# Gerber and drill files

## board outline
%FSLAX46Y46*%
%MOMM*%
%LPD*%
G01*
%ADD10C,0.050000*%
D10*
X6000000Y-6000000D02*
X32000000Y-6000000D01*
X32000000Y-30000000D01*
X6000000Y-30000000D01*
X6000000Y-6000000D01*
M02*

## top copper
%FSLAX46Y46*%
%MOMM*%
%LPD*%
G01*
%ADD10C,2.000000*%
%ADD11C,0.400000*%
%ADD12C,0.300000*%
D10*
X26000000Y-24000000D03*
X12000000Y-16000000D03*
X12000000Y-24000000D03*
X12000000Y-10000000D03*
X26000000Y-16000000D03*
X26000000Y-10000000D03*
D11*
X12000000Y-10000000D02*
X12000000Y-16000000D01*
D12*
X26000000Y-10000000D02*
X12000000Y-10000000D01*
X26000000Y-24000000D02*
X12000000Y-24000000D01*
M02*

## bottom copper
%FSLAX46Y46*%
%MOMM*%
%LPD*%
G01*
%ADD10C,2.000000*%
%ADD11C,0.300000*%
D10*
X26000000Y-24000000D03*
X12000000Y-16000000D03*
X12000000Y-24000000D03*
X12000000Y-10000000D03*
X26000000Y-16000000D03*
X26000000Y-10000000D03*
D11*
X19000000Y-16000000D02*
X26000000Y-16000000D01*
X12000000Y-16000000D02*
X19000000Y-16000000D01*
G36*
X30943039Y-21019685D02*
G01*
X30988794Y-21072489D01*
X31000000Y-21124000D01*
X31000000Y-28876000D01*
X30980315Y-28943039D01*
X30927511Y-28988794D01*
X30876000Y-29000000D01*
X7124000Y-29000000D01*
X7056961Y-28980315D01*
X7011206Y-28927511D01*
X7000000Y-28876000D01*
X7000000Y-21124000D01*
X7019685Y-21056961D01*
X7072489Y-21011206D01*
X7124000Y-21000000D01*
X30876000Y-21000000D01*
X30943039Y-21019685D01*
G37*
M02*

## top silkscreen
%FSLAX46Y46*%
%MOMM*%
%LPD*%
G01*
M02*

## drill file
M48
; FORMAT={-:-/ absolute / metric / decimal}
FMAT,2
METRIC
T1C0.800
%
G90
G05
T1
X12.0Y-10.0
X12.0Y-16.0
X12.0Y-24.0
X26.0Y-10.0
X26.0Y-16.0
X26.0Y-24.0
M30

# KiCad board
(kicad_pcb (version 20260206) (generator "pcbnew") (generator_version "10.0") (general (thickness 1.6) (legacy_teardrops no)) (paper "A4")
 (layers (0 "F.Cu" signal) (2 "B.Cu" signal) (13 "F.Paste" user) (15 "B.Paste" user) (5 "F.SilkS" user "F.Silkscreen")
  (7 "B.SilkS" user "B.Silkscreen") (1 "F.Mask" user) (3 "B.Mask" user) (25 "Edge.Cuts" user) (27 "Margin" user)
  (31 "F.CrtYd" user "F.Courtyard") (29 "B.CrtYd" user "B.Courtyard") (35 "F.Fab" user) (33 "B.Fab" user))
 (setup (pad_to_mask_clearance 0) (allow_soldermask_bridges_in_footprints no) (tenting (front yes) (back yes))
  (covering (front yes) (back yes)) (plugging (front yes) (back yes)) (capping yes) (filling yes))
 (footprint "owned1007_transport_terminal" (layer "F.Cu") (at 26 24)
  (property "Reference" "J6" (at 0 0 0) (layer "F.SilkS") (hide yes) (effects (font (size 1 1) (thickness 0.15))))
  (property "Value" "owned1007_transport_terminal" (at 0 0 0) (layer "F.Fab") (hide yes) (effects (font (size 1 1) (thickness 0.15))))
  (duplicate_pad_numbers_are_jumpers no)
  (pad "1" thru_hole circle (at 0 0) (size 2 2) (drill 0.8) (layers "*.Cu" "*.Mask") (remove_unused_layers no) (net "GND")))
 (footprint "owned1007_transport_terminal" (layer "F.Cu") (at 12 16)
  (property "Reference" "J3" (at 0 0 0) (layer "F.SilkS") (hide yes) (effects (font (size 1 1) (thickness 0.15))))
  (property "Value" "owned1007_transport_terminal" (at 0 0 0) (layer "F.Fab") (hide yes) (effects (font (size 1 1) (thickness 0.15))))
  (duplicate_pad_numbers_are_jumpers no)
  (pad "1" thru_hole circle (at 0 0) (size 2 2) (drill 0.8) (layers "*.Cu" "*.Mask") (remove_unused_layers no) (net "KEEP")))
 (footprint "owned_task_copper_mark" (layer "F.Cu") (at 10 28)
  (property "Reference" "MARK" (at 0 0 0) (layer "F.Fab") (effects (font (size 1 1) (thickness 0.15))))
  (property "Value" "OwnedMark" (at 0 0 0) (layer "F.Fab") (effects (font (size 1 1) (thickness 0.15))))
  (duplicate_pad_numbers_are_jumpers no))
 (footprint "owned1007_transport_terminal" (layer "F.Cu") (at 12 24)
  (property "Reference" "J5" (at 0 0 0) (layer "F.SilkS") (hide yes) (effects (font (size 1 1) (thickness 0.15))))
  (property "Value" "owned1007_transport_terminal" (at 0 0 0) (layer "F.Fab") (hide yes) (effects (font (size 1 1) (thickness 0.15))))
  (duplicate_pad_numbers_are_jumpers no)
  (pad "1" thru_hole circle (at 0 0) (size 2 2) (drill 0.8) (layers "*.Cu" "*.Mask") (remove_unused_layers no) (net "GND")))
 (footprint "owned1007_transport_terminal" (layer "F.Cu") (at 12 10)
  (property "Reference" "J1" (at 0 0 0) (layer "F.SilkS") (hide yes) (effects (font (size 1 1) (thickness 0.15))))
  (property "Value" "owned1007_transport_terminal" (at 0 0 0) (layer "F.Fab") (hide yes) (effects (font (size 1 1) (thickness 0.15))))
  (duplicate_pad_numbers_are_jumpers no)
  (pad "1" thru_hole circle (at 0 0) (size 2 2) (drill 0.8) (layers "*.Cu" "*.Mask") (remove_unused_layers no) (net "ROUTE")))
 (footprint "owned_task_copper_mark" (layer "F.Cu") (at 13 28)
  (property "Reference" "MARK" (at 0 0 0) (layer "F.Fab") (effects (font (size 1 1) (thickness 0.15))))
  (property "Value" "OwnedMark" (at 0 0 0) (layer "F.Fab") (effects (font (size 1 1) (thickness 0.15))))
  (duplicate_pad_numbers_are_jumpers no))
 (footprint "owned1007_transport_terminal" (layer "F.Cu") (at 26 16)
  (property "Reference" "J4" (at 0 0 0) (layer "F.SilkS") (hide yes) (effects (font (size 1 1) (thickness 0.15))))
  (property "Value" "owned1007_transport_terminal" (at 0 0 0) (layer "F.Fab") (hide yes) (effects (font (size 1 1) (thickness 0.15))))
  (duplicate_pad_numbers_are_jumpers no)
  (pad "1" thru_hole circle (at 0 0) (size 2 2) (drill 0.8) (layers "*.Cu" "*.Mask") (remove_unused_layers no) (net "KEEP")))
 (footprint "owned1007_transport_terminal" (layer "F.Cu") (at 26 10)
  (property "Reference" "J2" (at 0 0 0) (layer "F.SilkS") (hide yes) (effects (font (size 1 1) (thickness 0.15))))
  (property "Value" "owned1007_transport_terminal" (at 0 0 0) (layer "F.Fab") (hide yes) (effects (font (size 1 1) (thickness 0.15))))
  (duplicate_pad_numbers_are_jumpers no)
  (pad "1" thru_hole circle (at 0 0) (size 2 2) (drill 0.8) (layers "*.Cu" "*.Mask") (remove_unused_layers no) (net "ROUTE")))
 (gr_rect (start 6 6) (end 32 30) (stroke (width 0.05) (type default)) (fill no) (layer "Edge.Cuts"))
 (segment (start 12 10) (end 12 16) (width 0.4) (layer "F.Cu") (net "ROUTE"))
 (segment (start 26 10) (end 12 10) (width 0.3) (layer "F.Cu") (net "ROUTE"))
 (segment (start 19 16) (end 26 16) (width 0.3) (layer "B.Cu") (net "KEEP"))
 (segment (start 12 16) (end 19 16) (width 0.3) (locked yes) (layer "B.Cu") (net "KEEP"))
 (segment (start 26 24) (end 12 24) (width 0.3) (layer "F.Cu") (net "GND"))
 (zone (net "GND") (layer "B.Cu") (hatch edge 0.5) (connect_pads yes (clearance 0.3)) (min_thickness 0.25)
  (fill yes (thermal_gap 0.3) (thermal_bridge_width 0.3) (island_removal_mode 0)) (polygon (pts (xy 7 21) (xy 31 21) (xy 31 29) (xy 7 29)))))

